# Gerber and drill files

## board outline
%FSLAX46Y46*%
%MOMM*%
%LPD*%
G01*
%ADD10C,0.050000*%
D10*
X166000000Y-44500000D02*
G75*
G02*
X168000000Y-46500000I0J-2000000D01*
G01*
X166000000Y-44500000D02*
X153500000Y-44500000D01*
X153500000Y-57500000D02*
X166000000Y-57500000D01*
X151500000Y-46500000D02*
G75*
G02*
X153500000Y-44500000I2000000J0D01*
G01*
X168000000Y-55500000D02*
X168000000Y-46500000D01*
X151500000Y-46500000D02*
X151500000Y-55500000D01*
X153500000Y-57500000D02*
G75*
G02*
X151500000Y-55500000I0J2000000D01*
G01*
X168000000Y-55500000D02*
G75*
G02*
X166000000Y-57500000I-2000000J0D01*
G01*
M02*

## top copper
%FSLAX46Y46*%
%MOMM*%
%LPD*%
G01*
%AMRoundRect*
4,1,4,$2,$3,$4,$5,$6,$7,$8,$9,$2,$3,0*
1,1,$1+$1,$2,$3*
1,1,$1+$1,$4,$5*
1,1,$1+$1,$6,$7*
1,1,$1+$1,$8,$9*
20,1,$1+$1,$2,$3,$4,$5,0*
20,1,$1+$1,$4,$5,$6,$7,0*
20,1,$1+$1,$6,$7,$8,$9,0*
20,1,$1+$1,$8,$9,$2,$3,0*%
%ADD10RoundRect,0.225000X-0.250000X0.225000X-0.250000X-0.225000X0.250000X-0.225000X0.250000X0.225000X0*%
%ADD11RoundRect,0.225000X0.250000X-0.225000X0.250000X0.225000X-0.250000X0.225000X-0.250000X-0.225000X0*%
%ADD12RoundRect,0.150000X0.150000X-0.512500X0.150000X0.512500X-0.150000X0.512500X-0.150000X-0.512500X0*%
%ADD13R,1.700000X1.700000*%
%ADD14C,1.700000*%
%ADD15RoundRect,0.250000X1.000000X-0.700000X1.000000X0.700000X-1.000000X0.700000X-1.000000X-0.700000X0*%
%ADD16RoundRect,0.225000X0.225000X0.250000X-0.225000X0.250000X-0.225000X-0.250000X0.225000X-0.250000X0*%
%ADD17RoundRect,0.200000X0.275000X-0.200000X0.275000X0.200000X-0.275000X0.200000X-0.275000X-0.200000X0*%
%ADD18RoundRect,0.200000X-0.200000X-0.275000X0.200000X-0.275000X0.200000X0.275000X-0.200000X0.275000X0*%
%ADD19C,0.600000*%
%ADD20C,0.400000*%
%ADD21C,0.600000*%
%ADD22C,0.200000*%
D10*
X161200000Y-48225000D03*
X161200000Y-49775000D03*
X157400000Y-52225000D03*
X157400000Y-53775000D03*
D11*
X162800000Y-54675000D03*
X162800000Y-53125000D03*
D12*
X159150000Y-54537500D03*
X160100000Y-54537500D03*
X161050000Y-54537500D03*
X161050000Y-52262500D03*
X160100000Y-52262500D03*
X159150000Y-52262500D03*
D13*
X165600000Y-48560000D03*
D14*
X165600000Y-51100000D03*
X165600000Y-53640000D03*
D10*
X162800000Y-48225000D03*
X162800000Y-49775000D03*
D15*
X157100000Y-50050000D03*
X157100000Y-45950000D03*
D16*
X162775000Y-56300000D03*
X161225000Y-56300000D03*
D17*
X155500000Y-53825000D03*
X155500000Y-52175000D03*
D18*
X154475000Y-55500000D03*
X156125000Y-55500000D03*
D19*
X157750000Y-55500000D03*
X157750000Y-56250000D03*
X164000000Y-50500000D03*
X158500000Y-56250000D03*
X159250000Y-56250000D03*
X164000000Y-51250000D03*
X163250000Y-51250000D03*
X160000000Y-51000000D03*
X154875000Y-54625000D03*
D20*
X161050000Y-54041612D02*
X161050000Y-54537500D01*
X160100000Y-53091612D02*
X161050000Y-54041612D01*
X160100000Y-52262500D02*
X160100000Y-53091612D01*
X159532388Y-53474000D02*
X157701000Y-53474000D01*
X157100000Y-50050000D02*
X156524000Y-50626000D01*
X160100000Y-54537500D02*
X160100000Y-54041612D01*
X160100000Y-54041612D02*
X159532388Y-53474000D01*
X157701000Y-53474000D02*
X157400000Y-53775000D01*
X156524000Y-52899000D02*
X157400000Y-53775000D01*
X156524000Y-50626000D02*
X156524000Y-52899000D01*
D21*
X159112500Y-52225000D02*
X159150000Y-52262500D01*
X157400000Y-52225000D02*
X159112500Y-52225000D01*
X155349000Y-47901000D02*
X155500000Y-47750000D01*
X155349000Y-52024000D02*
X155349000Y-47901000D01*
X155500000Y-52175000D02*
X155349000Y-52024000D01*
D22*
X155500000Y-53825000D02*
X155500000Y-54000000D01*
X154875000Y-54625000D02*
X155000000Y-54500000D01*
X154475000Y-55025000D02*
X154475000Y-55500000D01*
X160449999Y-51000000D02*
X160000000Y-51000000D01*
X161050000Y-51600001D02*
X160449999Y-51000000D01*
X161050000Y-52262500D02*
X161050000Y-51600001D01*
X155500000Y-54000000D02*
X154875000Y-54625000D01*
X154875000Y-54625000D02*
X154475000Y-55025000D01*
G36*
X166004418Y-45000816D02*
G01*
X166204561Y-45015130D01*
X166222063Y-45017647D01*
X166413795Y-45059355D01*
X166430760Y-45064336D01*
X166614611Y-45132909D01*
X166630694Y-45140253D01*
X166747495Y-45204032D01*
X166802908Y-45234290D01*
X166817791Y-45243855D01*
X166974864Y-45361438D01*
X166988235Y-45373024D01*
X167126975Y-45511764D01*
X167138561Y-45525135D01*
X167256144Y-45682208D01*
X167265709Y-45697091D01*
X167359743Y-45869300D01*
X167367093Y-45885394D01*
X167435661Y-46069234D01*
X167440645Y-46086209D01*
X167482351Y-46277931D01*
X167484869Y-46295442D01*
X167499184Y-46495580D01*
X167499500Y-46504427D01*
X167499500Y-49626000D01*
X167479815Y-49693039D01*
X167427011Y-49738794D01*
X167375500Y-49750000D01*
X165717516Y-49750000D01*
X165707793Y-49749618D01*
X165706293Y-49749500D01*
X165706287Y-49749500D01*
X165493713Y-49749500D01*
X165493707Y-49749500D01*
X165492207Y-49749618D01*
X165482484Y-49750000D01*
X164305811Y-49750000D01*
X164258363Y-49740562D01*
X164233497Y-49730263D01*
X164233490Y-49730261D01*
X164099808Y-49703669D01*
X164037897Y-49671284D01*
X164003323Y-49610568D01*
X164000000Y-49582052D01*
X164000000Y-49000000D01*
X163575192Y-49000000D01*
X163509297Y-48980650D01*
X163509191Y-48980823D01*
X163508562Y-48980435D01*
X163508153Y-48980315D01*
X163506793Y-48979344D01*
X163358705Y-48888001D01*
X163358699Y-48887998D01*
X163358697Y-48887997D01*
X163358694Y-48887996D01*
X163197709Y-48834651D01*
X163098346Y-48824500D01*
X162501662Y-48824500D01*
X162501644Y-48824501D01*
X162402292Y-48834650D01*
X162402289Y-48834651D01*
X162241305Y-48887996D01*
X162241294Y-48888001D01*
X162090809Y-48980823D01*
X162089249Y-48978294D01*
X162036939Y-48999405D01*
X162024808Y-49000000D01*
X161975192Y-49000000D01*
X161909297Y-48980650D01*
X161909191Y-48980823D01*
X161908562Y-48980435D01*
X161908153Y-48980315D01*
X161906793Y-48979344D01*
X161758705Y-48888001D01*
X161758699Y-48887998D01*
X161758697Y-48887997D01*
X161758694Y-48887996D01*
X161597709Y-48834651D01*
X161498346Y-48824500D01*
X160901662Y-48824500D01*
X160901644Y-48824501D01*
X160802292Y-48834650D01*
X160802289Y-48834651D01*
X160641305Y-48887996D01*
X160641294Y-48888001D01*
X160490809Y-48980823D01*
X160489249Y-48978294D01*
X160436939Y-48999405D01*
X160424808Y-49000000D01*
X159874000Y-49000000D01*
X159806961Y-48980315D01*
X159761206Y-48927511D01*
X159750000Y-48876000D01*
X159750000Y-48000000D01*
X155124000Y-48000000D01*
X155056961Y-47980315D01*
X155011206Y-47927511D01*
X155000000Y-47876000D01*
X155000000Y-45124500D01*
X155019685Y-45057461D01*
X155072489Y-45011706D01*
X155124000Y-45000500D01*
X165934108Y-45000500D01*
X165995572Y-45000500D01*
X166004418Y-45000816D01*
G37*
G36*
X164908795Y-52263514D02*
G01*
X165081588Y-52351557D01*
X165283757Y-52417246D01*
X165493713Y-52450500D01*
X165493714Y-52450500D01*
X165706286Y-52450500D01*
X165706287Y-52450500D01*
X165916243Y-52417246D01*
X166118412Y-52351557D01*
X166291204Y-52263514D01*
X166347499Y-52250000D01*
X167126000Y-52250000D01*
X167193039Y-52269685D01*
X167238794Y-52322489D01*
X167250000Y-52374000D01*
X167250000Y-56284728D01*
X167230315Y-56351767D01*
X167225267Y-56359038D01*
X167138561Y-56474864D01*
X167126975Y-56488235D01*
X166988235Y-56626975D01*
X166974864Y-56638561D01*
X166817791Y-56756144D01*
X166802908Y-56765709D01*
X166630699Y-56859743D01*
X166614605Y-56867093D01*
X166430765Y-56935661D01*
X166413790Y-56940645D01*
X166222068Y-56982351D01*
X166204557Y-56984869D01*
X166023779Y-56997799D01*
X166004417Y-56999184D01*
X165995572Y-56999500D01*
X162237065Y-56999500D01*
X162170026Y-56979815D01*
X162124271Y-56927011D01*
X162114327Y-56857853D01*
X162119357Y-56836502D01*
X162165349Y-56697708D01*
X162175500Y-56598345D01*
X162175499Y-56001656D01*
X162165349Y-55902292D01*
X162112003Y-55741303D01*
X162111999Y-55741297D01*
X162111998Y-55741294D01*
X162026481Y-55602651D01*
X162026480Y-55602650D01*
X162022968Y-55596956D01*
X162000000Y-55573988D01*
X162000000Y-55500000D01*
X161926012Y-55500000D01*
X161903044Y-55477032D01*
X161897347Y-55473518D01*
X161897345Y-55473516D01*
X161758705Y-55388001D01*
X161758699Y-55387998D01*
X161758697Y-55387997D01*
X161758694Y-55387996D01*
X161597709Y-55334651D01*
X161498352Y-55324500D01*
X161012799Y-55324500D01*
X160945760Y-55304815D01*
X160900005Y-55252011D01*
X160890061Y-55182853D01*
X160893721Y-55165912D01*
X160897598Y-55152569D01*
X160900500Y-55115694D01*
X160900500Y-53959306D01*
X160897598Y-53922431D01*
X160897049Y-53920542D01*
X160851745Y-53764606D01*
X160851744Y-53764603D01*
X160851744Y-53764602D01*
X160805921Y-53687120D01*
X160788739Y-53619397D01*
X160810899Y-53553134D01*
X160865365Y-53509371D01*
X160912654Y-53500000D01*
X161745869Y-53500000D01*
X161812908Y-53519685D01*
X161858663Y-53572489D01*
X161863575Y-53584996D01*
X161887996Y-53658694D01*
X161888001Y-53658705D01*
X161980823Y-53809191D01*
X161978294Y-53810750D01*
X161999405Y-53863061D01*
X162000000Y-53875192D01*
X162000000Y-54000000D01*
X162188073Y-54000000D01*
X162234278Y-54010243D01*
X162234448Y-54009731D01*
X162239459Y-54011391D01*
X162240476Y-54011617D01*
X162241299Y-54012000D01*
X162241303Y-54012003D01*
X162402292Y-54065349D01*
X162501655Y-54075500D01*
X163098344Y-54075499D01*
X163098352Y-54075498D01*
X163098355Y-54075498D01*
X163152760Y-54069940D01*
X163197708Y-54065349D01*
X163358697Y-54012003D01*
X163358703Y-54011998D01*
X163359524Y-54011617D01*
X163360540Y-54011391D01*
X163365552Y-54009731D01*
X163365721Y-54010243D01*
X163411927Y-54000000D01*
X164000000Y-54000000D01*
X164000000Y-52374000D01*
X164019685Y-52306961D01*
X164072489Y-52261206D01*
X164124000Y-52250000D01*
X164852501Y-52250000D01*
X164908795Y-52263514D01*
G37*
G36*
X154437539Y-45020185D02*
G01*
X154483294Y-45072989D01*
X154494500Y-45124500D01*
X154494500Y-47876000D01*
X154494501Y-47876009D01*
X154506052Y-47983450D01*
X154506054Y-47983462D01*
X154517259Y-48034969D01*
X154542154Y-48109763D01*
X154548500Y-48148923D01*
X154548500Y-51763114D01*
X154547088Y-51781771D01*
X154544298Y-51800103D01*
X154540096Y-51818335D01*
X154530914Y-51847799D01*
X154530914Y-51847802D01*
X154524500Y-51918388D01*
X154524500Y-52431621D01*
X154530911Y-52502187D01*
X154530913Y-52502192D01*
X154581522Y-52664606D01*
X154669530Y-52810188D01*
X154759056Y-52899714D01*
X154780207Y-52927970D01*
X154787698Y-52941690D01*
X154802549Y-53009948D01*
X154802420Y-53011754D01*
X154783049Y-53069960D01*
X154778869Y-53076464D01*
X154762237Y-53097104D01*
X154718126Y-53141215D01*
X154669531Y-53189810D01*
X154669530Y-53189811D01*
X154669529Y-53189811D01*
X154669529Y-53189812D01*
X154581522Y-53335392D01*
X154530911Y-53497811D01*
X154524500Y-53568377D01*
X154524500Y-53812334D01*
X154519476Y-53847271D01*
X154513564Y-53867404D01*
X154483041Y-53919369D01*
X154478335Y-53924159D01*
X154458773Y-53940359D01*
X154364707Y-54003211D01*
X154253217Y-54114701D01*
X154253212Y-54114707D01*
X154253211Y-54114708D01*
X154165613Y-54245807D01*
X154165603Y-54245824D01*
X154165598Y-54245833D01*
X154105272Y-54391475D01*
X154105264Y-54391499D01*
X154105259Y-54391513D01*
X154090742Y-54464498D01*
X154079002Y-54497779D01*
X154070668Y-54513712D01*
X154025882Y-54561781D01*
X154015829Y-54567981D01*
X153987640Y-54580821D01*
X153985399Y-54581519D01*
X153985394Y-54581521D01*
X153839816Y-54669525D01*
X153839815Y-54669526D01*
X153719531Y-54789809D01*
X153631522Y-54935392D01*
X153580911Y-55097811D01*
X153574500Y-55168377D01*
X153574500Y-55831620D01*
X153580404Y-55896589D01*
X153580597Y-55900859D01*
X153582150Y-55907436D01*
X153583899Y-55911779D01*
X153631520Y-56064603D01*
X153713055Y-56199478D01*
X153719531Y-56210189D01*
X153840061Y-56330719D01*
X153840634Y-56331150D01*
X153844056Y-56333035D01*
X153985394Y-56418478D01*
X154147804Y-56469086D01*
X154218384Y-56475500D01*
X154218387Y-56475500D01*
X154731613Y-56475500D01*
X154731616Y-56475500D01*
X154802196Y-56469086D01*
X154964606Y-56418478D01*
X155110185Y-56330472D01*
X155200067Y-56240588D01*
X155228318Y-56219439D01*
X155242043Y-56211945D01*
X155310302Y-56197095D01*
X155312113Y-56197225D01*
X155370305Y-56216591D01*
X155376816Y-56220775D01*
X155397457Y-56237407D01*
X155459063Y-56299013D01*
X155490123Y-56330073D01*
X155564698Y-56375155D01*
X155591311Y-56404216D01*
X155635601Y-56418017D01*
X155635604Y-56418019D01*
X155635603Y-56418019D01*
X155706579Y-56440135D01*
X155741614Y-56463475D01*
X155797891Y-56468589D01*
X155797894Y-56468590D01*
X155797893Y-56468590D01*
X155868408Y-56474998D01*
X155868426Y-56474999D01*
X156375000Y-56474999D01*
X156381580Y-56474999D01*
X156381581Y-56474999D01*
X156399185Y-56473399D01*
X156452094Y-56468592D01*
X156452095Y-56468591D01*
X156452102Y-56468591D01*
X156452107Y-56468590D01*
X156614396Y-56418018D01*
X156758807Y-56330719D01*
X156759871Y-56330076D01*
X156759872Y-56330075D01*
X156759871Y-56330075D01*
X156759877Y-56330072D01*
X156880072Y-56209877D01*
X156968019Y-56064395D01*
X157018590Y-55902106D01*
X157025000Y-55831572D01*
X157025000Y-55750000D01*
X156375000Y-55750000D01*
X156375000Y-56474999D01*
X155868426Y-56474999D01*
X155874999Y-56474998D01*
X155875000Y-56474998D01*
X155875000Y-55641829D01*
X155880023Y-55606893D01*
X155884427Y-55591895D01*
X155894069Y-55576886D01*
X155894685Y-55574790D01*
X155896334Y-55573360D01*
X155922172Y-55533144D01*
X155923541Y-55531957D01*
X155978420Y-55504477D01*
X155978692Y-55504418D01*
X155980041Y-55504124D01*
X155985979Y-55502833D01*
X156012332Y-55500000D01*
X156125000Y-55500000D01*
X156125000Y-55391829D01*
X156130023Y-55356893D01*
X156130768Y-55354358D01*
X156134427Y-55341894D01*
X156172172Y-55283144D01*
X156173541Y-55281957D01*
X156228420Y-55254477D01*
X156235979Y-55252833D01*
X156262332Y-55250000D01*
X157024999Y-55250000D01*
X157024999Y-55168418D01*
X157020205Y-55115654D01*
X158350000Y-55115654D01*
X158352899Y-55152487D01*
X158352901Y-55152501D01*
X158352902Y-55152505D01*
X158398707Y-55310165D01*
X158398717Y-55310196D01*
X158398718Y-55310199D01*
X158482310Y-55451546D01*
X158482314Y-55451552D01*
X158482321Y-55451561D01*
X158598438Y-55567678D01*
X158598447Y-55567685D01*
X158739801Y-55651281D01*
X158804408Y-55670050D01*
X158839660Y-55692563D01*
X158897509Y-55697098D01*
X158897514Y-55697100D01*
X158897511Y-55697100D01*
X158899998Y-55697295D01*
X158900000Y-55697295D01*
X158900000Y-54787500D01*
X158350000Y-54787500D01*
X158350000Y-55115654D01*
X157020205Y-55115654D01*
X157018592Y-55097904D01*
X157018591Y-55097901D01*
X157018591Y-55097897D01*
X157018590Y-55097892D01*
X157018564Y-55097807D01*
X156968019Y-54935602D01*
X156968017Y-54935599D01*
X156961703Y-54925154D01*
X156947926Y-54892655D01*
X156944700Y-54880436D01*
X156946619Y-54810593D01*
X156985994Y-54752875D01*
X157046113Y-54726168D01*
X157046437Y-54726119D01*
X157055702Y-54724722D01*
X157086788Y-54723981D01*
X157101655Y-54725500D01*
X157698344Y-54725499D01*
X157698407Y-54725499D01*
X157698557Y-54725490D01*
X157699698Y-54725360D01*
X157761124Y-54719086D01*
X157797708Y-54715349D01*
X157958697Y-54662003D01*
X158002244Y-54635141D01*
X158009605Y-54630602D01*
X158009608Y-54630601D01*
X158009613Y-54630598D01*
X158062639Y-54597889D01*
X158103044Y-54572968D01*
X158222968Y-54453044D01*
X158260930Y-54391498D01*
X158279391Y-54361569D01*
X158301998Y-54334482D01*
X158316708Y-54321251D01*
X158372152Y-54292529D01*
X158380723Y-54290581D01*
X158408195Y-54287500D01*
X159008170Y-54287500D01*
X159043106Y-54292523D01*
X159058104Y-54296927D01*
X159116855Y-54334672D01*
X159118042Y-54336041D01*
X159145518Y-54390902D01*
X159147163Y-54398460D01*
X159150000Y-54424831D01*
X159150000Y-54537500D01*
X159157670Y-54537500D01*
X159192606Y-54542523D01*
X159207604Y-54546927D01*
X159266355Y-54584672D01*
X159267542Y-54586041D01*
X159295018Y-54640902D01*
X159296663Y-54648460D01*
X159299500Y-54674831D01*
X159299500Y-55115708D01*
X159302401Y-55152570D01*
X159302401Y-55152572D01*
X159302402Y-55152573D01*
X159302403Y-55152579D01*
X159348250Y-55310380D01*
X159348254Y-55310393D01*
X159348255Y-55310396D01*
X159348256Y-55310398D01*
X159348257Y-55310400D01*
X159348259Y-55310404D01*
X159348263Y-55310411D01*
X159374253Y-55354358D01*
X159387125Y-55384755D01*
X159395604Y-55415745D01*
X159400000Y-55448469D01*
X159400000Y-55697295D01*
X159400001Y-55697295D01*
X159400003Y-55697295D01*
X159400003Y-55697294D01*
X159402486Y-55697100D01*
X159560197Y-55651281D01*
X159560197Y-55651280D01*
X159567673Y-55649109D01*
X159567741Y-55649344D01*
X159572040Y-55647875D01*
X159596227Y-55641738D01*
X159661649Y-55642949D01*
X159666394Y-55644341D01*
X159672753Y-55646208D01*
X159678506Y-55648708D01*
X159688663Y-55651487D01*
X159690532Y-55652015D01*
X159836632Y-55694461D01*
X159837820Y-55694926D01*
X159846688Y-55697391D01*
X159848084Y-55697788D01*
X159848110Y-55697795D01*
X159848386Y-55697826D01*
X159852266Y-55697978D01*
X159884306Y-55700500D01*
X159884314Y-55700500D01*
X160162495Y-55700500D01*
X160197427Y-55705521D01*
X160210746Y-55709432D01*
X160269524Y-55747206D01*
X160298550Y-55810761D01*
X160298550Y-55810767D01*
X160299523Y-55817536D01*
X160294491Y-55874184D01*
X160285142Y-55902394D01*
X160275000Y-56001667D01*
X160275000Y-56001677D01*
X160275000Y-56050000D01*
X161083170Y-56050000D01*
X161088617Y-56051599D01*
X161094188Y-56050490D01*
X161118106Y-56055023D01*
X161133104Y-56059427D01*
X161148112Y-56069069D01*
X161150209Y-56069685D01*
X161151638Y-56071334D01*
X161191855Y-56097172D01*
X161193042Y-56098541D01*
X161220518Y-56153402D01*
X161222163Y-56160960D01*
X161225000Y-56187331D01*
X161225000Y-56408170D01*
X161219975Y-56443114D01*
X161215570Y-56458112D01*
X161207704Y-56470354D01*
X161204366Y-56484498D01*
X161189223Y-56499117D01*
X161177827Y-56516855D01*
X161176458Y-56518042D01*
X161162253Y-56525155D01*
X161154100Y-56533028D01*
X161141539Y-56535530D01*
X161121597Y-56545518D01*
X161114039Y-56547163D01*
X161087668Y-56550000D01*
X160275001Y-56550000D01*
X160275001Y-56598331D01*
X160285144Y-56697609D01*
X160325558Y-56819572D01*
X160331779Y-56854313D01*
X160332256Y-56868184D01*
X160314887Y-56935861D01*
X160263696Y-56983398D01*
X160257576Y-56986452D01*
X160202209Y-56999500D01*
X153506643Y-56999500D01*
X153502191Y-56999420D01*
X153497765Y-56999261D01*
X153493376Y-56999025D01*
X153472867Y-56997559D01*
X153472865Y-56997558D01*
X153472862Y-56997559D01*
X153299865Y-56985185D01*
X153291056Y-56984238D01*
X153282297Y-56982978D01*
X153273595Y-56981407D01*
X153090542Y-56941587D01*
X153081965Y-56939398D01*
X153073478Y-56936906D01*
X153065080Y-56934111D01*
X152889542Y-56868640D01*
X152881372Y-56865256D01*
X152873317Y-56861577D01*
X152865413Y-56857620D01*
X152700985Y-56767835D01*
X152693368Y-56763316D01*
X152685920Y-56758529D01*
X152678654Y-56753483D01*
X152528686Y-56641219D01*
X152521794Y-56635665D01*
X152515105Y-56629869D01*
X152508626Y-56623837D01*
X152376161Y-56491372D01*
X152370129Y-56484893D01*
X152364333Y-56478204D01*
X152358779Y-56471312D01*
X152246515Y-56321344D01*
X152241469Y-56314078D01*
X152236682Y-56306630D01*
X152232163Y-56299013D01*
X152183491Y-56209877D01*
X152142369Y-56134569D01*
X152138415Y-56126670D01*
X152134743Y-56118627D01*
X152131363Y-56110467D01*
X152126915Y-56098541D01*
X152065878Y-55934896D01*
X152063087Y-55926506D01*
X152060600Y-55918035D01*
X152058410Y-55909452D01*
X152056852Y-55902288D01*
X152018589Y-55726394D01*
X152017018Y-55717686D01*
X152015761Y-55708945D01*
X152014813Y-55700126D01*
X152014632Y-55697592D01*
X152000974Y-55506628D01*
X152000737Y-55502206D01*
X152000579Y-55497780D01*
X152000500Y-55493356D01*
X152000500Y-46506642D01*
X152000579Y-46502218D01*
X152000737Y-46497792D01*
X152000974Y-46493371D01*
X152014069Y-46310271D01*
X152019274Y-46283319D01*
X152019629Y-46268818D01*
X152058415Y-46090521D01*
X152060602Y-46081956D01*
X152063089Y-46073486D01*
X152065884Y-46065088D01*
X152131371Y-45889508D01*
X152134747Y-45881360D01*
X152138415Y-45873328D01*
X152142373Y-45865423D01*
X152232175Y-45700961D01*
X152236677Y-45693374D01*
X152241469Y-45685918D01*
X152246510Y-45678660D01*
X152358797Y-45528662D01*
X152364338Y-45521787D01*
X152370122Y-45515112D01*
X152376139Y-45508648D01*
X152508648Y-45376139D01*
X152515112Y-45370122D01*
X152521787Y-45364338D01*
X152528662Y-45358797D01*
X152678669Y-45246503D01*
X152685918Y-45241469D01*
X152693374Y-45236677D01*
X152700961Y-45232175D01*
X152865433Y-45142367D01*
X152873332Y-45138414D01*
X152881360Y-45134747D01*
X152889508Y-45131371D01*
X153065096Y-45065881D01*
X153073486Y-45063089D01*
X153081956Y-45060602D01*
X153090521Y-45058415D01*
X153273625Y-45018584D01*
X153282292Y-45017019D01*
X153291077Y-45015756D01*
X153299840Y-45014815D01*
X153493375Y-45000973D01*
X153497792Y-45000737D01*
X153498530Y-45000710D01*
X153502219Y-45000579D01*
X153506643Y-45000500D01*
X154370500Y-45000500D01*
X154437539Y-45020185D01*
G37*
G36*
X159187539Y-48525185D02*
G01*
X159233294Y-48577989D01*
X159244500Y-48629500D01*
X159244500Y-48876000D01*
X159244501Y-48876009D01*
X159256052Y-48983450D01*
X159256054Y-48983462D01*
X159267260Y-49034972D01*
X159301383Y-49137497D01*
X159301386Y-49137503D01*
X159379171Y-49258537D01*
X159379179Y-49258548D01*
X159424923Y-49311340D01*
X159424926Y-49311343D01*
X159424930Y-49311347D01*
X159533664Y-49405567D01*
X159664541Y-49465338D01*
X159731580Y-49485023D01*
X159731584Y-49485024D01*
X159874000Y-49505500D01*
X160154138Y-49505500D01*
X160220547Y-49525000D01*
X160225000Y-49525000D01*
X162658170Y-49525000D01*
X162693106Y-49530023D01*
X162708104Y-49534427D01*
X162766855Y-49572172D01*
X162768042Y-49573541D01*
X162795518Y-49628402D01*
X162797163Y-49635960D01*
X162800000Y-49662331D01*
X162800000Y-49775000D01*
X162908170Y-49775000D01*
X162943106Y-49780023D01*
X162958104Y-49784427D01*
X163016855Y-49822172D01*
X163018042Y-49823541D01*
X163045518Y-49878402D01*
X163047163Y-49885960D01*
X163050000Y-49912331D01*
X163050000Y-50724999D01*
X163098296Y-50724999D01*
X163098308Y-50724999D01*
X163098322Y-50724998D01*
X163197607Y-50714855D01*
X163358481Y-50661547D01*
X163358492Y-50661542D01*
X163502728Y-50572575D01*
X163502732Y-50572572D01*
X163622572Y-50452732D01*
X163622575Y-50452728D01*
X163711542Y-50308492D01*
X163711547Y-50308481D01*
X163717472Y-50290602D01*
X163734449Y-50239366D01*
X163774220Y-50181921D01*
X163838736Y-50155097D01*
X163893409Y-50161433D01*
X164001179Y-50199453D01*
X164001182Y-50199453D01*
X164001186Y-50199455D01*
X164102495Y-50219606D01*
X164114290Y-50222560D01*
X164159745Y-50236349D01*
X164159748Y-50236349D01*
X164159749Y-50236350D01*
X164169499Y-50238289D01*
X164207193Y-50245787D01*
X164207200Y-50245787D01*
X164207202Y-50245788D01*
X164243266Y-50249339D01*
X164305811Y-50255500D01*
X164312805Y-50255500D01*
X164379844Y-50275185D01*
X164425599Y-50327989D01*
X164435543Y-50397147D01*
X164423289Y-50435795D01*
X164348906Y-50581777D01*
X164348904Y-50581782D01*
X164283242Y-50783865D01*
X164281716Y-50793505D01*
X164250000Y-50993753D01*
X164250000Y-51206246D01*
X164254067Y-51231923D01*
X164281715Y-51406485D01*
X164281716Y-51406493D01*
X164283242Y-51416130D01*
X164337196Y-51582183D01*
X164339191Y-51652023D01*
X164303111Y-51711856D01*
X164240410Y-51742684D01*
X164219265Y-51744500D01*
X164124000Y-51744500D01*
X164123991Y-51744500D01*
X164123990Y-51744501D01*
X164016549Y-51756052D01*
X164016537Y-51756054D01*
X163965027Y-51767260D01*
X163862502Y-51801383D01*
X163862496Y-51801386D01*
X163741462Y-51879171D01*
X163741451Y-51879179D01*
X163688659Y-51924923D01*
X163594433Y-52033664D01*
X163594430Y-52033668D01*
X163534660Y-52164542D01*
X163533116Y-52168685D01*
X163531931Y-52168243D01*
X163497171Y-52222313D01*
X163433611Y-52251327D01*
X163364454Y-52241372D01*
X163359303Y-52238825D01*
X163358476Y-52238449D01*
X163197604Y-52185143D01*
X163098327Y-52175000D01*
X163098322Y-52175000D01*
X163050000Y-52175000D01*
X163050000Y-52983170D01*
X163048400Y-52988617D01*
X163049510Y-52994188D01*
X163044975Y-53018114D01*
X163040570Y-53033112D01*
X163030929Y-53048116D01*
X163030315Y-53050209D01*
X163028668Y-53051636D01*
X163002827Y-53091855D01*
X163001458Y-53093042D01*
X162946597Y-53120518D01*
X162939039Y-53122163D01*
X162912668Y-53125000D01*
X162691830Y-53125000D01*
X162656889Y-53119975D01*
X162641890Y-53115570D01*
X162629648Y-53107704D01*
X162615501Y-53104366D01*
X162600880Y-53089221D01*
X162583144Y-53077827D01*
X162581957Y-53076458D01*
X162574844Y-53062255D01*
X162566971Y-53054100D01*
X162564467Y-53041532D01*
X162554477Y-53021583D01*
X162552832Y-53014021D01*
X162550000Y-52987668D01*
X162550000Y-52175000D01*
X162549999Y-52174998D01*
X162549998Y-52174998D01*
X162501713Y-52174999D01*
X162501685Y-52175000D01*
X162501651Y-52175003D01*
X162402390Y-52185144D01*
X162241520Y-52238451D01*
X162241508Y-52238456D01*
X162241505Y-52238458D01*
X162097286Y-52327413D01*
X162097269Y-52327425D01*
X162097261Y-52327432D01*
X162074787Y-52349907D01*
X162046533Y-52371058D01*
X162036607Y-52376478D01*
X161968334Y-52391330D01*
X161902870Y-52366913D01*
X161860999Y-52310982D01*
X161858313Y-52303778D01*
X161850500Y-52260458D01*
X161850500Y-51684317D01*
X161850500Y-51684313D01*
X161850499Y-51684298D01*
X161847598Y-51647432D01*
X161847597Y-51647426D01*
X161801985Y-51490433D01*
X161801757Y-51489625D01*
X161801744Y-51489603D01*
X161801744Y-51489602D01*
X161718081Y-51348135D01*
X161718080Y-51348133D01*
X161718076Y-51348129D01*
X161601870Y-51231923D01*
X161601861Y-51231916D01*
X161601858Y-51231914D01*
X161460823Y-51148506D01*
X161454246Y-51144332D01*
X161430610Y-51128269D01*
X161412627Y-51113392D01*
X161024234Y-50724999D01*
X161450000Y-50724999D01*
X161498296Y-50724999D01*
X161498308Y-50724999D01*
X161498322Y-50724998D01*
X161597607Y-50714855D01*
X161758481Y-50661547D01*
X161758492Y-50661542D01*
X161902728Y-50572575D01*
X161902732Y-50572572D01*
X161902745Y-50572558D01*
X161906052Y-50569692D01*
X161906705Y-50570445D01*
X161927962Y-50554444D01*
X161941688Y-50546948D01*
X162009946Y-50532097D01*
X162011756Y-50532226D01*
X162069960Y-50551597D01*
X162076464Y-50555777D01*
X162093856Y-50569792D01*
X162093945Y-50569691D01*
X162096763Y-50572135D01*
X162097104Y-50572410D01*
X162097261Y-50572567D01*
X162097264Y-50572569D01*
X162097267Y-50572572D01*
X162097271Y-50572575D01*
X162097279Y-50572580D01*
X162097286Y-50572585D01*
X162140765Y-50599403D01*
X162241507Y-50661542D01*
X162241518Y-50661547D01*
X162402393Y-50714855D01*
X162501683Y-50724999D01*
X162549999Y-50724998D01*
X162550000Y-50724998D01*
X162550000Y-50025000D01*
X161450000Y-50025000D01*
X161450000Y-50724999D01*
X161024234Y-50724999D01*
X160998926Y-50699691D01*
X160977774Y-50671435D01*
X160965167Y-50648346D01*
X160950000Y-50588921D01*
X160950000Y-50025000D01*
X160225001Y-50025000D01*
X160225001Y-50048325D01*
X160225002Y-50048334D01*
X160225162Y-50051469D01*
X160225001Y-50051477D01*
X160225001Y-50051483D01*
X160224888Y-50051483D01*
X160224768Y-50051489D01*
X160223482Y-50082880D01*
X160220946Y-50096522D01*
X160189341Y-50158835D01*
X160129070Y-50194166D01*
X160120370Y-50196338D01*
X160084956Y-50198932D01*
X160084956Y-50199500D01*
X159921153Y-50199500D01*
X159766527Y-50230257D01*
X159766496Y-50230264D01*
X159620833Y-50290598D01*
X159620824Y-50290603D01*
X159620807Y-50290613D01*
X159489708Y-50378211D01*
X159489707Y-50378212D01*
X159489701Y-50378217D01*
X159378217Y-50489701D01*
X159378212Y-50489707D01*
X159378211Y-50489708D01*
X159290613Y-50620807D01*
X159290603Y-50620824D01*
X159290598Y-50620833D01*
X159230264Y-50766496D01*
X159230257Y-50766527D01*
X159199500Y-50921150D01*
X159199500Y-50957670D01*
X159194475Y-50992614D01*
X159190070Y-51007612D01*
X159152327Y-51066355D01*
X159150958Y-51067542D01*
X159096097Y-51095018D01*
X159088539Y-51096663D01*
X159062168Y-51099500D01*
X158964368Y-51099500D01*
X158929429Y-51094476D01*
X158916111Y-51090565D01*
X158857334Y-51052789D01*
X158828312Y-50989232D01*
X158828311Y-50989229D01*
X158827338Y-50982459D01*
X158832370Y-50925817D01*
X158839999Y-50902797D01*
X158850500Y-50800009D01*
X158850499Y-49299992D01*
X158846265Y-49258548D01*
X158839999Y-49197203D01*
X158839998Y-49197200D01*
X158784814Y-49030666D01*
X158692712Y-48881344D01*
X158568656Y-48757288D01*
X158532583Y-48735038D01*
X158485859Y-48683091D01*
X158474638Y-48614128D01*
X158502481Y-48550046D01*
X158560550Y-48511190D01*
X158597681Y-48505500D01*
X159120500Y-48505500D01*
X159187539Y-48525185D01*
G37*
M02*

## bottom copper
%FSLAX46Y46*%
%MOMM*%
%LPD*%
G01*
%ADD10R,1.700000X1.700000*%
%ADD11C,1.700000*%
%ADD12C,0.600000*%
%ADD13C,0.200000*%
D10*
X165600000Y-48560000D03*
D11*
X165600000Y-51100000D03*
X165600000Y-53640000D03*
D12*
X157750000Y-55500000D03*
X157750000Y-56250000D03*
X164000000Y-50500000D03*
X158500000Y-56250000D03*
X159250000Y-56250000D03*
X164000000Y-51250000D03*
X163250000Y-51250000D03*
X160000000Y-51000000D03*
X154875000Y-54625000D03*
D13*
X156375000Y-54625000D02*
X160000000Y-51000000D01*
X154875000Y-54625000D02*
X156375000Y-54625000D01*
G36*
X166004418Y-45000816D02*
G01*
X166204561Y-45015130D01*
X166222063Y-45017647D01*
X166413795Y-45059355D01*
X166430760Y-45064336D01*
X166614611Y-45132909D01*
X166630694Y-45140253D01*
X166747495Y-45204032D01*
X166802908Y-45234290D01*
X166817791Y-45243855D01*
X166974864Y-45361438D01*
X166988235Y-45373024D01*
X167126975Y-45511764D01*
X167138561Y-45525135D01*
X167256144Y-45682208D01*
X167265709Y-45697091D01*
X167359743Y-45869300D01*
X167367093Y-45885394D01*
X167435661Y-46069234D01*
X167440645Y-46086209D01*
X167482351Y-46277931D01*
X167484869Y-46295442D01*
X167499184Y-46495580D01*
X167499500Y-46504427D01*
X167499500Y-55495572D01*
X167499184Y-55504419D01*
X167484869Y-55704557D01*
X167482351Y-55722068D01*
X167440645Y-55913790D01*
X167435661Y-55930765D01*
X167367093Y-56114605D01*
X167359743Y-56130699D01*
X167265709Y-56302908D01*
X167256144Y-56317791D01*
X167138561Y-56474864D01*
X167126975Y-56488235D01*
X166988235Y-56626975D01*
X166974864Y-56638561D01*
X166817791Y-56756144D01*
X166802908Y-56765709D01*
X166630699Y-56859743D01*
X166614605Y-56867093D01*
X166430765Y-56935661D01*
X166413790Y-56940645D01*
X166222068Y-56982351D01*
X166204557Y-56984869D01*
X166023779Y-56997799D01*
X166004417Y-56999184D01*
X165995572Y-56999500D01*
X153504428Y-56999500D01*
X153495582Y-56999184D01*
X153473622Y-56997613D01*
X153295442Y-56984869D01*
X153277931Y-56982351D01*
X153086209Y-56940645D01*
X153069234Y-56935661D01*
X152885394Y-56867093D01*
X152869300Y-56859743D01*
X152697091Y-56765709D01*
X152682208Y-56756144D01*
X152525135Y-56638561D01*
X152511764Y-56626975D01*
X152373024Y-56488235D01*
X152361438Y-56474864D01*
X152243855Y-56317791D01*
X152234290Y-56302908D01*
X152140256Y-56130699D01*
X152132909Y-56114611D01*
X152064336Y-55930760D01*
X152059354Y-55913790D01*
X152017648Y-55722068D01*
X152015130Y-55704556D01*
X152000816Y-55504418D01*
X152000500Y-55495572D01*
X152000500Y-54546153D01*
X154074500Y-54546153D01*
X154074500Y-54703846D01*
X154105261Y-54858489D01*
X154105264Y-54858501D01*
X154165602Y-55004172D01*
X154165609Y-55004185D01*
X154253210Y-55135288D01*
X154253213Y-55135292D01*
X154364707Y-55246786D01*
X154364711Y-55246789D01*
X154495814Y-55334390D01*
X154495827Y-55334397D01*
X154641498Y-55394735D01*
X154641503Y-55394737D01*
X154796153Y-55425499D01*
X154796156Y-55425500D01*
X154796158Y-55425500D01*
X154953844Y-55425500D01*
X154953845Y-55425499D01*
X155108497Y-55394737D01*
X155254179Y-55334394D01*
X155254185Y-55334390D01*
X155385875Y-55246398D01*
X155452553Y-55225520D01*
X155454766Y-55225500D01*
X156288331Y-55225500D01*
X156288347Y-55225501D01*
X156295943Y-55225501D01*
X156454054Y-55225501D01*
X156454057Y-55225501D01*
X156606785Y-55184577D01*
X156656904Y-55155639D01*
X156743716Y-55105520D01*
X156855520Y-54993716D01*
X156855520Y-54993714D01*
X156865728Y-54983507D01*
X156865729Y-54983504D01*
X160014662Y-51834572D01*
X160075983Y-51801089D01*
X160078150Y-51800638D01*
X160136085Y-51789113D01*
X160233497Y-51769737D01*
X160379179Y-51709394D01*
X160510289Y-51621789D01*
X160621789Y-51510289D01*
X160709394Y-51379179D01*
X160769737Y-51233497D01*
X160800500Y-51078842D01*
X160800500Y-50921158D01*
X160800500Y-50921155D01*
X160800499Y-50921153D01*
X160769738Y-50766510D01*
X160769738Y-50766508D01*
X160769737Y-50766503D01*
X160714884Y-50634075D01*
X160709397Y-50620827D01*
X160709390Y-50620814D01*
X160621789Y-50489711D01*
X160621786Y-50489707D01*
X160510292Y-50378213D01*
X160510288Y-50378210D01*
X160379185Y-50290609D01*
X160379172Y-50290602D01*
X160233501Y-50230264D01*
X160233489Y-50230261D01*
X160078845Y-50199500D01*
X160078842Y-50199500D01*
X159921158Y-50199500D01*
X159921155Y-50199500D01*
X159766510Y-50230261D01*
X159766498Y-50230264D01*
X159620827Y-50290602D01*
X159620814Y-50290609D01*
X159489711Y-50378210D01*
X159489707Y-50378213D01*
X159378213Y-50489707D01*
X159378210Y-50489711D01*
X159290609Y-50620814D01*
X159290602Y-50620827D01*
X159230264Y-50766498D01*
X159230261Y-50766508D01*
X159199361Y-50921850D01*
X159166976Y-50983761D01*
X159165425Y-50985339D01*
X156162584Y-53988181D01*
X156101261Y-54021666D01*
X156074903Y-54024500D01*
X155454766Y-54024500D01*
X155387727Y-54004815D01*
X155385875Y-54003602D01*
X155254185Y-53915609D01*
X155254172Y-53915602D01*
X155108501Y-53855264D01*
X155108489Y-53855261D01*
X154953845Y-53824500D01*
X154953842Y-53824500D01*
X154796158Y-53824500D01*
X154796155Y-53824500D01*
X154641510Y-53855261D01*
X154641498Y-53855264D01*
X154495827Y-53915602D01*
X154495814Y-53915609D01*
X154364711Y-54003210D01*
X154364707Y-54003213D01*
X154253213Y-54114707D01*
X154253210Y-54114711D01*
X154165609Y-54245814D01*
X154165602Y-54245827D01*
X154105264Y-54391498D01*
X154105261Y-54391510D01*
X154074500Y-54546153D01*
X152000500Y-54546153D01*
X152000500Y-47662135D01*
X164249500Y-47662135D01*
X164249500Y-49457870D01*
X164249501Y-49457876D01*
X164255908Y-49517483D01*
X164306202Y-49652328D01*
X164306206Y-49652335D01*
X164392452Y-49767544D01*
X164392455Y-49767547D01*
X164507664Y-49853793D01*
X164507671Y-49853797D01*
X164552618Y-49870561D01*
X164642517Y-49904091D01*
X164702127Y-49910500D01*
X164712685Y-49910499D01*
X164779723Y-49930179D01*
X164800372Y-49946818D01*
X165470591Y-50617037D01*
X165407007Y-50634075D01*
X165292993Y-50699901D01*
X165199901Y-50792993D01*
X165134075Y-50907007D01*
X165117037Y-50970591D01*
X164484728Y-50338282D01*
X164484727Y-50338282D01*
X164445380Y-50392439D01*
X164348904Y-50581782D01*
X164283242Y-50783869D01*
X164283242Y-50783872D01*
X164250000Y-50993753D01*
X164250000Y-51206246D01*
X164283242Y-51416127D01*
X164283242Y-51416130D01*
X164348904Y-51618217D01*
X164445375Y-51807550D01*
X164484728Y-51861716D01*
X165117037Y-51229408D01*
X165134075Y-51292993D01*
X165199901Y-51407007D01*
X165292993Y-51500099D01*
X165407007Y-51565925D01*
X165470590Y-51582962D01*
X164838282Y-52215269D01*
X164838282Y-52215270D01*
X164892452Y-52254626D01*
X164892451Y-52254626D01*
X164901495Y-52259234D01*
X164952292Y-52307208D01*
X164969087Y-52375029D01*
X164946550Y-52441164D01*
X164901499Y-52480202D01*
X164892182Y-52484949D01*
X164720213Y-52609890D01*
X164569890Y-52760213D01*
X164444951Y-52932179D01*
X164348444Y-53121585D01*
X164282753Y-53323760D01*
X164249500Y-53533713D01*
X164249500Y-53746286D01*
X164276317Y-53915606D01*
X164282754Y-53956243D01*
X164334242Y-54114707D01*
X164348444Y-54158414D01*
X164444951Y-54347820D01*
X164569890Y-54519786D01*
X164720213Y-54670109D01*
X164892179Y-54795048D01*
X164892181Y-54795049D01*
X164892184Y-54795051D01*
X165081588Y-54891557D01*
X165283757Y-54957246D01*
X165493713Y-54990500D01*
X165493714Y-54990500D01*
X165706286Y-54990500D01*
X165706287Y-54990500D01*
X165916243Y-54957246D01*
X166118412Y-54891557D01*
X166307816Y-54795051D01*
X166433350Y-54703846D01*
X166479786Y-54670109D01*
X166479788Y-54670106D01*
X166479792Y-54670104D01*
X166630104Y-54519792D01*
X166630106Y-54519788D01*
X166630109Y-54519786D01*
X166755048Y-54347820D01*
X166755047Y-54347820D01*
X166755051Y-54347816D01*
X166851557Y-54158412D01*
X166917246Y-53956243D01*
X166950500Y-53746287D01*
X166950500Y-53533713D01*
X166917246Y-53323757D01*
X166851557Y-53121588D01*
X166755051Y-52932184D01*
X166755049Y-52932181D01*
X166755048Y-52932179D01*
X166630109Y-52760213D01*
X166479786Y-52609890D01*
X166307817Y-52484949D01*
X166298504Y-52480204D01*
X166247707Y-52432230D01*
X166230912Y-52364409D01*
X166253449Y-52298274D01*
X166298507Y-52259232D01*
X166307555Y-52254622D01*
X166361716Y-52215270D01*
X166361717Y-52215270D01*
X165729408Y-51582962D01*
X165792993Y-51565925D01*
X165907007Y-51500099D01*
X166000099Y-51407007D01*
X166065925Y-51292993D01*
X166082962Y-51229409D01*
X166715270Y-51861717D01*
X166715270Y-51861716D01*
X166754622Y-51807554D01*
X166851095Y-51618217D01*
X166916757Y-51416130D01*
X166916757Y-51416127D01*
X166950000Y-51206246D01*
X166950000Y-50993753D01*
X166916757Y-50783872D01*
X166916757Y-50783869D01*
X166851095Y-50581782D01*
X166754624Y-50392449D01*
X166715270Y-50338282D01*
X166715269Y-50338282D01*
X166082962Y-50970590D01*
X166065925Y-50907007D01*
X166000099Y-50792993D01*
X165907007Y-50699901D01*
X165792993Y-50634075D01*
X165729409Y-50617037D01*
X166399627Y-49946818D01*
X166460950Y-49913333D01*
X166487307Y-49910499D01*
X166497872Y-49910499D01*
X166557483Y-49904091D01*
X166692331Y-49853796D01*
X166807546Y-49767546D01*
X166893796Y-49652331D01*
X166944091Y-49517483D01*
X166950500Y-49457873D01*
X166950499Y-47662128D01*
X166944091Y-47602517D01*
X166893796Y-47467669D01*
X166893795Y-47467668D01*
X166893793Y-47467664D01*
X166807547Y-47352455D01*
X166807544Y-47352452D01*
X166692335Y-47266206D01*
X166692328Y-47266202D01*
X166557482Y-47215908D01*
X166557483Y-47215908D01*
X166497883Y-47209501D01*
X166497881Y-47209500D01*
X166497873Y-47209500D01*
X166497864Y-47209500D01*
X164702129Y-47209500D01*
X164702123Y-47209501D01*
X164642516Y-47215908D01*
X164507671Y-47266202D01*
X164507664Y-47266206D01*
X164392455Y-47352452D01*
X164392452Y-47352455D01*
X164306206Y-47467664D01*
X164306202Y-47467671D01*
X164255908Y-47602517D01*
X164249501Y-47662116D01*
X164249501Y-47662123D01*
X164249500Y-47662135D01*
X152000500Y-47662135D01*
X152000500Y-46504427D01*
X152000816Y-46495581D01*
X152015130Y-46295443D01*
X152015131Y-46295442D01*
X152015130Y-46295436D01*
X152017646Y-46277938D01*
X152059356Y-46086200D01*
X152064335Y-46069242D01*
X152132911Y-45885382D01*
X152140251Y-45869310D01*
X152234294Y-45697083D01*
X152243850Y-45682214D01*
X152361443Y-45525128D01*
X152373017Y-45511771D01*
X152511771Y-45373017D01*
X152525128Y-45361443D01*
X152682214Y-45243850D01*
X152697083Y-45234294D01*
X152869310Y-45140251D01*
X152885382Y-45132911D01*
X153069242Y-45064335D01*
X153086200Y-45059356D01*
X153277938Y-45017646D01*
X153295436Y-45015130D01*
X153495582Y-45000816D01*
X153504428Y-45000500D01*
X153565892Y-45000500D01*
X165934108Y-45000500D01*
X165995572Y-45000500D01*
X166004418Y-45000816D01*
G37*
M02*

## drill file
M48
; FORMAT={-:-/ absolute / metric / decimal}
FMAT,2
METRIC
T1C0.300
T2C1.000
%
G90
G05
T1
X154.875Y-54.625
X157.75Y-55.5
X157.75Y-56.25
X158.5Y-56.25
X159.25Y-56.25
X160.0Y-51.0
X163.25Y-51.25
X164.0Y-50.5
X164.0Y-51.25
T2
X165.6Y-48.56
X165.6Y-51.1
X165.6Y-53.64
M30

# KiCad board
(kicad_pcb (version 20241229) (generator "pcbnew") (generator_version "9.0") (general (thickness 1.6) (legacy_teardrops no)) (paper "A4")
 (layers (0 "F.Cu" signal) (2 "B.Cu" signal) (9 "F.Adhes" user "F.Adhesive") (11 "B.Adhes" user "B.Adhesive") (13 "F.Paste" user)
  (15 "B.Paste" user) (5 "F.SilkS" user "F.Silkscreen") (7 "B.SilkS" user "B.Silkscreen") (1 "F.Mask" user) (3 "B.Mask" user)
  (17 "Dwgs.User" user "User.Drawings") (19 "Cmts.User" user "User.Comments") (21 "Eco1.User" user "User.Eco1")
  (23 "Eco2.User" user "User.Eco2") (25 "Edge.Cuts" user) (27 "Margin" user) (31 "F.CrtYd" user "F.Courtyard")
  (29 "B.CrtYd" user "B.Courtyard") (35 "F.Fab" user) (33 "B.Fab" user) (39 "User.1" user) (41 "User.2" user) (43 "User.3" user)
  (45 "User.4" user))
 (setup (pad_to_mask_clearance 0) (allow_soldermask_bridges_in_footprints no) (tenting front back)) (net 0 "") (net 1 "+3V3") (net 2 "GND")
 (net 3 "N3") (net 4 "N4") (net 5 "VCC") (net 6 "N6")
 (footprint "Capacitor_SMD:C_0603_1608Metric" (layer "F.Cu") (at 161.2 49 -90)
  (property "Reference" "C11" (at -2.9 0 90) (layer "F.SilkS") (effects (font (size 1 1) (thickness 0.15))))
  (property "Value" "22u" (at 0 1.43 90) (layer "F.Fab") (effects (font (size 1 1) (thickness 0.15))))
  (pad "1" smd roundrect (at -0.775 0 270) (size 0.9 0.95) (layers "F.Cu" "F.Mask" "F.Paste") (roundrect_rratio 0.25) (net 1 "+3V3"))
  (pad "2" smd roundrect (at 0.775 0 270) (size 0.9 0.95) (layers "F.Cu" "F.Mask" "F.Paste") (roundrect_rratio 0.25) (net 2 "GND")))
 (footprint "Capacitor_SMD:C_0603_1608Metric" (layer "F.Cu") (at 157.4 53 -90)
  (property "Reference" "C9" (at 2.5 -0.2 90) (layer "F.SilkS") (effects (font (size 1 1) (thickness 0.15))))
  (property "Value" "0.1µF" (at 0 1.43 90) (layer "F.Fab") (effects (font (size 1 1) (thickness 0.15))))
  (pad "1" smd roundrect (at -0.775 0 270) (size 0.9 0.95) (layers "F.Cu" "F.Mask" "F.Paste") (roundrect_rratio 0.25) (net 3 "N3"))
  (pad "2" smd roundrect (at 0.775 0 270) (size 0.9 0.95) (layers "F.Cu" "F.Mask" "F.Paste") (roundrect_rratio 0.25) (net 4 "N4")))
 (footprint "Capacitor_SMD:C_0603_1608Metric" (layer "F.Cu") (at 162.8 53.9 90)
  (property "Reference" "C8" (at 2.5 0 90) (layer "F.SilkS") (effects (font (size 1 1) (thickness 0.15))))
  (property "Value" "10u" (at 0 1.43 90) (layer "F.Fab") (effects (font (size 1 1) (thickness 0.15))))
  (pad "1" smd roundrect (at -0.775 0 90) (size 0.9 0.95) (layers "F.Cu" "F.Mask" "F.Paste") (roundrect_rratio 0.25) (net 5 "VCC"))
  (pad "2" smd roundrect (at 0.775 0 90) (size 0.9 0.95) (layers "F.Cu" "F.Mask" "F.Paste") (roundrect_rratio 0.25) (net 2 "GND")))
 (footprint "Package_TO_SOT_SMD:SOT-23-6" (layer "F.Cu") (at 160.1 53.4 90)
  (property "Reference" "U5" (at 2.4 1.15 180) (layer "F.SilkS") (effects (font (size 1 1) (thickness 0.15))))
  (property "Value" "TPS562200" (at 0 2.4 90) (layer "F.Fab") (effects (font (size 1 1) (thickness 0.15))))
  (pad "1" smd roundrect (at -1.1375 -0.95 90) (size 1.325 0.6) (layers "F.Cu" "F.Mask" "F.Paste") (roundrect_rratio 0.25) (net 2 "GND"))
  (pad "2" smd roundrect (at -1.1375 0 90) (size 1.325 0.6) (layers "F.Cu" "F.Mask" "F.Paste") (roundrect_rratio 0.25) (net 4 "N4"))
  (pad "3" smd roundrect (at -1.1375 0.95 90) (size 1.325 0.6) (layers "F.Cu" "F.Mask" "F.Paste") (roundrect_rratio 0.25) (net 5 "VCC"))
  (pad "4" smd roundrect (at 1.1375 0.95 90) (size 1.325 0.6) (layers "F.Cu" "F.Mask" "F.Paste") (roundrect_rratio 0.25) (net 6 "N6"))
  (pad "5" smd roundrect (at 1.1375 0 90) (size 1.325 0.6) (layers "F.Cu" "F.Mask" "F.Paste") (roundrect_rratio 0.25) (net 5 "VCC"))
  (pad "6" smd roundrect (at 1.1375 -0.95 90) (size 1.325 0.6) (layers "F.Cu" "F.Mask" "F.Paste") (roundrect_rratio 0.25) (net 3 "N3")))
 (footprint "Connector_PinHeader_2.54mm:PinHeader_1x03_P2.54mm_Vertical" (layer "F.Cu") (at 165.6 48.56)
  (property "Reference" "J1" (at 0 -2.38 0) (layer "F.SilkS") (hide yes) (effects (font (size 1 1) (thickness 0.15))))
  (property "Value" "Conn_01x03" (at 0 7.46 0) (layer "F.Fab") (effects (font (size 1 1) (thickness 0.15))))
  (pad "1" thru_hole rect (at 0 0) (size 1.7 1.7) (drill 1) (layers "*.Cu" "*.Mask") (remove_unused_layers no) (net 1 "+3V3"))
  (pad "2" thru_hole circle (at 0 2.54) (size 1.7 1.7) (drill 1) (layers "*.Cu" "*.Mask") (remove_unused_layers no) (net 2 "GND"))
  (pad "3" thru_hole circle (at 0 5.08) (size 1.7 1.7) (drill 1) (layers "*.Cu" "*.Mask") (remove_unused_layers no) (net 5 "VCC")))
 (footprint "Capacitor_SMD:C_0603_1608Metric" (layer "F.Cu") (at 162.8 49 -90)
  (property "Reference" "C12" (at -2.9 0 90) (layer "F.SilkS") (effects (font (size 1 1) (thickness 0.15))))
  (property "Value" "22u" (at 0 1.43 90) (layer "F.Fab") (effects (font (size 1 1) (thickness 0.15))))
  (pad "1" smd roundrect (at -0.775 0 270) (size 0.9 0.95) (layers "F.Cu" "F.Mask" "F.Paste") (roundrect_rratio 0.25) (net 1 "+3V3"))
  (pad "2" smd roundrect (at 0.775 0 270) (size 0.9 0.95) (layers "F.Cu" "F.Mask" "F.Paste") (roundrect_rratio 0.25) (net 2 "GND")))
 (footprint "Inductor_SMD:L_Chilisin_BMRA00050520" (layer "F.Cu") (at 157.1 48 90)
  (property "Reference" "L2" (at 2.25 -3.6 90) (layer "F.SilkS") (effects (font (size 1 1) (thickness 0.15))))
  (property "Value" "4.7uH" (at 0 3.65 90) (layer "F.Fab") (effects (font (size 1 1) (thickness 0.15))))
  (pad "1" smd roundrect (at -2.05 0 90) (size 1.9 2.5) (layers "F.Cu" "F.Mask" "F.Paste") (roundrect_rratio 0.131579) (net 4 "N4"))
  (pad "2" smd roundrect (at 2.05 0 90) (size 1.9 2.5) (layers "F.Cu" "F.Mask" "F.Paste") (roundrect_rratio 0.131579) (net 1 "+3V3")))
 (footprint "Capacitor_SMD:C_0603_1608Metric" (layer "F.Cu") (at 162 56.3 180)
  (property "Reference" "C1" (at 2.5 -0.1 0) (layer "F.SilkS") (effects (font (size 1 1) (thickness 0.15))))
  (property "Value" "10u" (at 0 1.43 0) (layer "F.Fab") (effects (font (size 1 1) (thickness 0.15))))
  (pad "1" smd roundrect (at -0.775 0 180) (size 0.9 0.95) (layers "F.Cu" "F.Mask" "F.Paste") (roundrect_rratio 0.25) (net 5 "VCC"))
  (pad "2" smd roundrect (at 0.775 0 180) (size 0.9 0.95) (layers "F.Cu" "F.Mask" "F.Paste") (roundrect_rratio 0.25) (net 2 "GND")))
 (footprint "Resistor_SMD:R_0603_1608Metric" (layer "F.Cu") (at 155.5 53 90)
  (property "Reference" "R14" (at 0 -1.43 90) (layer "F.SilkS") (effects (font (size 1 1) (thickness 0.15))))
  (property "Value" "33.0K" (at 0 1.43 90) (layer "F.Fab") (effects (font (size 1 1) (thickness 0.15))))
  (pad "1" smd roundrect (at -0.825 0 90) (size 0.8 0.95) (layers "F.Cu" "F.Mask" "F.Paste") (roundrect_rratio 0.25) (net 6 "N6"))
  (pad "2" smd roundrect (at 0.825 0 90) (size 0.8 0.95) (layers "F.Cu" "F.Mask" "F.Paste") (roundrect_rratio 0.25) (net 1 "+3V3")))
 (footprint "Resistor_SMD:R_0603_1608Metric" (layer "F.Cu") (at 155.3 55.5)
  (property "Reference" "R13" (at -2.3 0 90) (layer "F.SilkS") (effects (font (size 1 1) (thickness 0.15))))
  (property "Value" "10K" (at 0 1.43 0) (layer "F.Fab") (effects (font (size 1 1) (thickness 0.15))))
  (pad "1" smd roundrect (at -0.825 0) (size 0.8 0.95) (layers "F.Cu" "F.Mask" "F.Paste") (roundrect_rratio 0.25) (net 6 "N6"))
  (pad "2" smd roundrect (at 0.825 0) (size 0.8 0.95) (layers "F.Cu" "F.Mask" "F.Paste") (roundrect_rratio 0.25) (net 2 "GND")))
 (gr_arc (start 166 44.5) (mid 167.414214 45.085786) (end 168 46.5) (stroke (width 0.05) (type default)) (layer "Edge.Cuts"))
 (gr_line (start 166 44.5) (end 153.5 44.5) (stroke (width 0.05) (type default)) (layer "Edge.Cuts"))
 (gr_line (start 153.5 57.5) (end 166 57.5) (stroke (width 0.05) (type default)) (layer "Edge.Cuts"))
 (gr_arc (start 151.5 46.5) (mid 152.085786 45.085786) (end 153.5 44.5) (stroke (width 0.05) (type default)) (layer "Edge.Cuts"))
 (gr_line (start 168 55.5) (end 168 46.5) (stroke (width 0.05) (type default)) (layer "Edge.Cuts"))
 (gr_line (start 151.5 46.5) (end 151.5 55.5) (stroke (width 0.05) (type default)) (layer "Edge.Cuts"))
 (gr_arc (start 153.5 57.5) (mid 152.085786 56.914214) (end 151.5 55.5) (stroke (width 0.05) (type default)) (layer "Edge.Cuts"))
 (gr_arc (start 168 55.5) (mid 167.414214 56.914214) (end 166 57.5) (stroke (width 0.05) (type default)) (layer "Edge.Cuts"))
 (via (at 157.75 55.5) (size 0.6) (drill 0.3) (layers "F.Cu" "B.Cu") (free yes) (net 2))
 (via (at 157.75 56.25) (size 0.6) (drill 0.3) (layers "F.Cu" "B.Cu") (free yes) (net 2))
 (via (at 164 50.5) (size 0.6) (drill 0.3) (layers "F.Cu" "B.Cu") (free yes) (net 2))
 (via (at 158.5 56.25) (size 0.6) (drill 0.3) (layers "F.Cu" "B.Cu") (free yes) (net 2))
 (via (at 159.25 56.25) (size 0.6) (drill 0.3) (layers "F.Cu" "B.Cu") (free yes) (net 2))
 (via (at 164 51.25) (size 0.6) (drill 0.3) (layers "F.Cu" "B.Cu") (free yes) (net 2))
 (via (at 163.25 51.25) (size 0.6) (drill 0.3) (layers "F.Cu" "B.Cu") (free yes) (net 2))
 (segment (start 161.05 54.041612) (end 161.05 54.5375) (width 0.4) (layer "F.Cu") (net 5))
 (segment (start 160.1 53.091612) (end 161.05 54.041612) (width 0.4) (layer "F.Cu") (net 5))
 (segment (start 160.1 52.2625) (end 160.1 53.091612) (width 0.4) (layer "F.Cu") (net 5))
 (segment (start 159.532388 53.474) (end 157.701 53.474) (width 0.4) (layer "F.Cu") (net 4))
 (segment (start 157.1 50.05) (end 156.524 50.626) (width 0.4) (layer "F.Cu") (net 4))
 (segment (start 160.1 54.5375) (end 160.1 54.041612) (width 0.4) (layer "F.Cu") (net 4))
 (segment (start 160.1 54.041612) (end 159.532388 53.474) (width 0.4) (layer "F.Cu") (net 4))
 (segment (start 157.701 53.474) (end 157.4 53.775) (width 0.4) (layer "F.Cu") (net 4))
 (segment (start 156.524 52.899) (end 157.4 53.775) (width 0.4) (layer "F.Cu") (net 4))
 (segment (start 156.524 50.626) (end 156.524 52.899) (width 0.4) (layer "F.Cu") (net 4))
 (segment (start 159.1125 52.225) (end 159.15 52.2625) (width 0.6) (layer "F.Cu") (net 3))
 (segment (start 157.4 52.225) (end 159.1125 52.225) (width 0.6) (layer "F.Cu") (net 3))
 (segment (start 155.349 47.901) (end 155.5 47.75) (width 0.6) (layer "F.Cu") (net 1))
 (segment (start 155.349 52.024) (end 155.349 47.901) (width 0.6) (layer "F.Cu") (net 1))
 (segment (start 155.5 52.175) (end 155.349 52.024) (width 0.6) (layer "F.Cu") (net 1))
 (segment (start 155.5 53.825) (end 155.5 54) (width 0.2) (layer "F.Cu") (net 6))
 (segment (start 154.875 54.625) (end 155 54.5) (width 0.2) (layer "F.Cu") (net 6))
 (segment (start 154.475 55.025) (end 154.475 55.5) (width 0.2) (layer "F.Cu") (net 6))
 (segment (start 160.449999 51) (end 160 51) (width 0.2) (layer "F.Cu") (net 6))
 (segment (start 161.05 51.600001) (end 160.449999 51) (width 0.2) (layer "F.Cu") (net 6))
 (segment (start 161.05 52.2625) (end 161.05 51.600001) (width 0.2) (layer "F.Cu") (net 6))
 (segment (start 155.5 54) (end 154.875 54.625) (width 0.2) (layer "F.Cu") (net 6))
 (segment (start 154.875 54.625) (end 154.475 55.025) (width 0.2) (layer "F.Cu") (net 6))
 (via (at 160 51) (size 0.6) (drill 0.3) (layers "F.Cu" "B.Cu") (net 6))
 (via (at 154.875 54.625) (size 0.6) (drill 0.3) (layers "F.Cu" "B.Cu") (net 6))
 (segment (start 156.375 54.625) (end 160 51) (width 0.2) (layer "B.Cu") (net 6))
 (segment (start 154.875 54.625) (end 156.375 54.625) (width 0.2) (layer "B.Cu") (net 6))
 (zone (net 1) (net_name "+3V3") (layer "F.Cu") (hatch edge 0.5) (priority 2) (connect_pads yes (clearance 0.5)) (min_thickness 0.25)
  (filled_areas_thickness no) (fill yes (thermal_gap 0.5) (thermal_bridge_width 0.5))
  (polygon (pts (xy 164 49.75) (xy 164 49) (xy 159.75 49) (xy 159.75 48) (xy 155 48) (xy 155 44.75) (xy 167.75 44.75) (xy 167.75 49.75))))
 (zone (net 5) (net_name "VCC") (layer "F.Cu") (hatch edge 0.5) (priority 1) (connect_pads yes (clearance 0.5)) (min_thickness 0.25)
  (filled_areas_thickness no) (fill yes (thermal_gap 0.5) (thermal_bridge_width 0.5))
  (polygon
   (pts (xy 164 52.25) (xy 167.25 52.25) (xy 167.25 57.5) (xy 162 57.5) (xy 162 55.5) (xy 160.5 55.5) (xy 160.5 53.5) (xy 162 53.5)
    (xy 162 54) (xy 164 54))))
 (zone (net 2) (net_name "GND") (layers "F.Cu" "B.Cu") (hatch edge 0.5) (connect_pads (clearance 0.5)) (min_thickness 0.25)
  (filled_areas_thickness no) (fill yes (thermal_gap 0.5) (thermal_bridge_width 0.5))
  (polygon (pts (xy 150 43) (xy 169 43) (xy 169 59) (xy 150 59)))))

